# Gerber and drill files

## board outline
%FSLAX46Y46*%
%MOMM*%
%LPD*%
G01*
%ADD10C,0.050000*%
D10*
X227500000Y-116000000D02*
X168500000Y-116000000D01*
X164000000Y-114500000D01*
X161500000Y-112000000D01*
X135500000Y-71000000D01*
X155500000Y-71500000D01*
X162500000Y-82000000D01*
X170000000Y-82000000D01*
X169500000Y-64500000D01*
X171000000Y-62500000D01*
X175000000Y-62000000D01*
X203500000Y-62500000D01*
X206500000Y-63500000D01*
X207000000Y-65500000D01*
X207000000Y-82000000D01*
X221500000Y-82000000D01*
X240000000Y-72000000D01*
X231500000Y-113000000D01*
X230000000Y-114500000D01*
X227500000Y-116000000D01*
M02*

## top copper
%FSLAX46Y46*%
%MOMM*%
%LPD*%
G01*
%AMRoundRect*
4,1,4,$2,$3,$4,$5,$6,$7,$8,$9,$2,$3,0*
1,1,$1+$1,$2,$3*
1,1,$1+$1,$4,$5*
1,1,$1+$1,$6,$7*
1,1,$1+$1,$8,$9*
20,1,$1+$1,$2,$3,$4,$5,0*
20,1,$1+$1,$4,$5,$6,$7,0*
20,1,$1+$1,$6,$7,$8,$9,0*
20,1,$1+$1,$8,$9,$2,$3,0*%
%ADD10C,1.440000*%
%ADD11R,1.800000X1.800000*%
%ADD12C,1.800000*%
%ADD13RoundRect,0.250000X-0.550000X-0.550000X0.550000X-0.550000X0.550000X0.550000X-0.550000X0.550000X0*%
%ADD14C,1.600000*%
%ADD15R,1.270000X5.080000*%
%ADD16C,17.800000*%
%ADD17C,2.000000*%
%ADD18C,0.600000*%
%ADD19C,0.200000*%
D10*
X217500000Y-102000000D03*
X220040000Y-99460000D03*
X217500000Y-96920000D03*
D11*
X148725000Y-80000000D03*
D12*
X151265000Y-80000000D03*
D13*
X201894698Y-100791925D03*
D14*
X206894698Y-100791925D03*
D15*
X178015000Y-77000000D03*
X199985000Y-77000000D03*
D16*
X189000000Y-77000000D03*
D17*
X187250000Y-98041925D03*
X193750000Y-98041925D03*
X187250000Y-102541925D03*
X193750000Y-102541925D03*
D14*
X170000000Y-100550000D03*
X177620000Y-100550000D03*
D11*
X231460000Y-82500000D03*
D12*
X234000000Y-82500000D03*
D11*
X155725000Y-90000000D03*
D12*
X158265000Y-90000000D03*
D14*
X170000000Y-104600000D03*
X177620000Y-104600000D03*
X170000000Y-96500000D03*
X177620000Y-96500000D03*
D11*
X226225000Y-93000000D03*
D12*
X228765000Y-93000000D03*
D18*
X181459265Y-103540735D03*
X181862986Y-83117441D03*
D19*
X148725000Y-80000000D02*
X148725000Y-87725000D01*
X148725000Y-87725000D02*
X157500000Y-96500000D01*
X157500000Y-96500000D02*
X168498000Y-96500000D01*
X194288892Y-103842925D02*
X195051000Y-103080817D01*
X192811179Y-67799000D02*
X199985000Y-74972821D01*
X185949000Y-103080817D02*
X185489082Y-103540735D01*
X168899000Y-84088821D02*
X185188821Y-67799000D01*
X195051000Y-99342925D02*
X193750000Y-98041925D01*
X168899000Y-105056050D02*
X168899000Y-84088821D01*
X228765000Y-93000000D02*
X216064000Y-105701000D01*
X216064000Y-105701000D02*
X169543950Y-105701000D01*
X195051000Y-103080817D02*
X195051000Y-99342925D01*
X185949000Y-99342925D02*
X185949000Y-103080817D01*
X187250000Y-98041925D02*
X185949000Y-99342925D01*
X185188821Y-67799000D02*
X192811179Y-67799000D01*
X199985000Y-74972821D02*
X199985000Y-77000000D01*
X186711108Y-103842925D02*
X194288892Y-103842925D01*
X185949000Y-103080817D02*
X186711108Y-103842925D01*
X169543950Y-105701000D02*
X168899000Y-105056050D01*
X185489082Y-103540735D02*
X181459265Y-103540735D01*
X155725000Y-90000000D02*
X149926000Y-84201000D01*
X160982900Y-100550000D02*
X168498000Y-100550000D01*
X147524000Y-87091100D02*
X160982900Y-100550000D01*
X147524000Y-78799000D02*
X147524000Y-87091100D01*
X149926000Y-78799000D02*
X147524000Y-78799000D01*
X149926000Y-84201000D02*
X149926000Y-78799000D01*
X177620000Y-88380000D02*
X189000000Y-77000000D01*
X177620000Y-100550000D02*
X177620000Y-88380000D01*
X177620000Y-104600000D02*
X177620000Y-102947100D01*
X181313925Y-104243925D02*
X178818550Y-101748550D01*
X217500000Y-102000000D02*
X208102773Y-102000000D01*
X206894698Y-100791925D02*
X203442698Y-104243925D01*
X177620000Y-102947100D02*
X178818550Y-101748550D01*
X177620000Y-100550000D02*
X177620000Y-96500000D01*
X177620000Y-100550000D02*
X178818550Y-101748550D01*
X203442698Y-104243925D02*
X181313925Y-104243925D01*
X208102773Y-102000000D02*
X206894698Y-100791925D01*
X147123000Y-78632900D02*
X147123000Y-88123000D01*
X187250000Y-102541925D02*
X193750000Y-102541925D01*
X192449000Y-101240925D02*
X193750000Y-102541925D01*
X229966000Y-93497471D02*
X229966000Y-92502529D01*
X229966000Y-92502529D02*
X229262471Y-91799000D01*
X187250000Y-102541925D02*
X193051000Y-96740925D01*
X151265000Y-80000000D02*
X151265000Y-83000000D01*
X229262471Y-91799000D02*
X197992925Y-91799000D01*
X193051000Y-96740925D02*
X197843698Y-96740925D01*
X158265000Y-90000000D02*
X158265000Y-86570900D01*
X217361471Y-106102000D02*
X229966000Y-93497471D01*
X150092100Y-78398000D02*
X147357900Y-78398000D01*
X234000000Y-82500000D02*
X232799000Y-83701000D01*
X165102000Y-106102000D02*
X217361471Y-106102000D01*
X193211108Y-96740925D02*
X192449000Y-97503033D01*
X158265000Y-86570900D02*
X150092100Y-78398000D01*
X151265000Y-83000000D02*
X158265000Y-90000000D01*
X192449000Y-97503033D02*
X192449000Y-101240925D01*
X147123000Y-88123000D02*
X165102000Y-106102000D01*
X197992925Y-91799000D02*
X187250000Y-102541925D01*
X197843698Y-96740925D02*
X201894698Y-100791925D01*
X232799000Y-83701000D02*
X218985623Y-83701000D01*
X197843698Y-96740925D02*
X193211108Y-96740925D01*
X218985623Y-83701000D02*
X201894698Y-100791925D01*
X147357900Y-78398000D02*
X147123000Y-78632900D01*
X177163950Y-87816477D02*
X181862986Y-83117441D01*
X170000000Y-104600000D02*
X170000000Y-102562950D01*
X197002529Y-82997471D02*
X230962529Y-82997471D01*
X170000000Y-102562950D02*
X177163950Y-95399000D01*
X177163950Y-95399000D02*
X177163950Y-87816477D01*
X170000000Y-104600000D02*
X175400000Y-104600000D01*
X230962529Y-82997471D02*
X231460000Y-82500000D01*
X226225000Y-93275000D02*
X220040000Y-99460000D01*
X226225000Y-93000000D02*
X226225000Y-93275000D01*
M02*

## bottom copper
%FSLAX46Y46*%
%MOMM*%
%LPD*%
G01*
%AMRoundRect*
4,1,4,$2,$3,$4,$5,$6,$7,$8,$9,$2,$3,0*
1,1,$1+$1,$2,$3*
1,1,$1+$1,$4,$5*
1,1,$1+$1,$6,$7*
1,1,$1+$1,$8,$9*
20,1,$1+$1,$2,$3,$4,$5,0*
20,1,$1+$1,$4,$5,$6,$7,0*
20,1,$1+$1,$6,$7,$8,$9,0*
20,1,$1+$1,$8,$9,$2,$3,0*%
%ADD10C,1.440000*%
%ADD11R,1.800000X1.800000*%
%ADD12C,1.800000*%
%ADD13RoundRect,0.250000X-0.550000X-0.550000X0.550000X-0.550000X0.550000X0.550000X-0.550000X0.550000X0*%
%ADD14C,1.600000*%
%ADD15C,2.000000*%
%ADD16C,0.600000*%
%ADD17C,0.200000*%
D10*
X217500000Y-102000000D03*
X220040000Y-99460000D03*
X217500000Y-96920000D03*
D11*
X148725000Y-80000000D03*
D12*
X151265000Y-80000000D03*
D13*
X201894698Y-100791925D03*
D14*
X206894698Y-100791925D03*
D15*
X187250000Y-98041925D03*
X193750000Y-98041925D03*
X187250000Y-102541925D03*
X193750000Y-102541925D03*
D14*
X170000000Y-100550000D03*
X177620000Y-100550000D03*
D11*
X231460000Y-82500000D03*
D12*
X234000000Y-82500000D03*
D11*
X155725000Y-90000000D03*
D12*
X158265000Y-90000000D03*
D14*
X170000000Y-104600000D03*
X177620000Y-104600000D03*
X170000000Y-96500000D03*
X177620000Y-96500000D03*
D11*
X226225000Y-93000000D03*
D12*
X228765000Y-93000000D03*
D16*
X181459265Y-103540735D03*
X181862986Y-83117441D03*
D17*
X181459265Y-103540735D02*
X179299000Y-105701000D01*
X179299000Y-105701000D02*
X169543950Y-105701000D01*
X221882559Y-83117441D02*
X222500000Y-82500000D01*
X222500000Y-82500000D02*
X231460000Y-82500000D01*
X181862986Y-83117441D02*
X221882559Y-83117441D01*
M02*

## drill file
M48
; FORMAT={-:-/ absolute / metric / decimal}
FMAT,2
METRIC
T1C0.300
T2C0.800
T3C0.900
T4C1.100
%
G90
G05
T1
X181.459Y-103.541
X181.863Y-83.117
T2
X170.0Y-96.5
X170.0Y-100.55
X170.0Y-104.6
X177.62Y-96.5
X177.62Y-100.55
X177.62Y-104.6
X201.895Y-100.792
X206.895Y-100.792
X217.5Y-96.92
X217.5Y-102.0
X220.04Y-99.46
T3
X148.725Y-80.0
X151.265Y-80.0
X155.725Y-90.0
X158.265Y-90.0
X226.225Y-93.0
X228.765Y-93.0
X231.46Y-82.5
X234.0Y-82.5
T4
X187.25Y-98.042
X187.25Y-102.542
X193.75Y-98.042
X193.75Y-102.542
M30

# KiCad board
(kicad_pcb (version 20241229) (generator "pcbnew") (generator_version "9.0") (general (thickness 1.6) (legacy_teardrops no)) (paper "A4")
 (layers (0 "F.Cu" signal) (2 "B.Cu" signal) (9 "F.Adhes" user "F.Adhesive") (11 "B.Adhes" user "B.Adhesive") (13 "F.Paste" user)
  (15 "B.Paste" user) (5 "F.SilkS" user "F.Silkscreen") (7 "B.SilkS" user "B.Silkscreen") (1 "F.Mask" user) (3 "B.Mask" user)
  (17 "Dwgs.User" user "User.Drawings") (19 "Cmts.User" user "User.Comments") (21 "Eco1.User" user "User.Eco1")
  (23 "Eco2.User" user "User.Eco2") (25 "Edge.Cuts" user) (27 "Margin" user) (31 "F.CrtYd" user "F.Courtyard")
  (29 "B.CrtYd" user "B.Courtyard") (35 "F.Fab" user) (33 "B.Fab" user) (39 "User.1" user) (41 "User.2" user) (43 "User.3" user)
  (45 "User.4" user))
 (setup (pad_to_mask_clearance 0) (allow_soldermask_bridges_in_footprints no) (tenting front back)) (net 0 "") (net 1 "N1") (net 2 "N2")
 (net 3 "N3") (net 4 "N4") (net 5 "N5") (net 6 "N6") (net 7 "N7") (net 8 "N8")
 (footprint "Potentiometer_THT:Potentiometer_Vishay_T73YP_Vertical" (layer "F.Cu") (at 217.5 102)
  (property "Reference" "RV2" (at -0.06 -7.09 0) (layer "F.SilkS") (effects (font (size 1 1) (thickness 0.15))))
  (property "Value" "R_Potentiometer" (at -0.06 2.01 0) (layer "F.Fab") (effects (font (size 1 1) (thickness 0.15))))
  (pad "1" thru_hole circle (at 0 0) (size 1.44 1.44) (drill 0.8) (layers "*.Cu" "*.Mask") (remove_unused_layers no) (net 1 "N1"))
  (pad "2" thru_hole circle (at 2.54 -2.54) (size 1.44 1.44) (drill 0.8) (layers "*.Cu" "*.Mask") (remove_unused_layers no) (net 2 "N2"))
  (pad "3" thru_hole circle (at 0 -5.08) (size 1.44 1.44) (drill 0.8) (layers "*.Cu" "*.Mask") (remove_unused_layers no) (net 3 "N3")))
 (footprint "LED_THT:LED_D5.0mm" (layer "F.Cu") (at 148.725 80)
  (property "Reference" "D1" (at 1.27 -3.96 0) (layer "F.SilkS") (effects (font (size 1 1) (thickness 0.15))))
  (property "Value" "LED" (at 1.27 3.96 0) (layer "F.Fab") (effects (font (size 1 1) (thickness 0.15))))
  (pad "1" thru_hole rect (at 0 0) (size 1.8 1.8) (drill 0.9) (layers "*.Cu" "*.Mask") (remove_unused_layers no) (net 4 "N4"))
  (pad "2" thru_hole circle (at 2.54 0) (size 1.8 1.8) (drill 0.9) (layers "*.Cu" "*.Mask") (remove_unused_layers no) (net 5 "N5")))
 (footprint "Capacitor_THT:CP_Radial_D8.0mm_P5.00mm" (layer "F.Cu") (at 201.894698 100.791925)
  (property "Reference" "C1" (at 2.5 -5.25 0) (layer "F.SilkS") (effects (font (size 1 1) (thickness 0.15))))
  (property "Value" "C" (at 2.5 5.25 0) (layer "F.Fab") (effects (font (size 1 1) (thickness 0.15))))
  (pad "1" thru_hole roundrect (at 0 0) (size 1.6 1.6) (drill 0.8) (layers "*.Cu" "*.Mask") (remove_unused_layers no)
   (roundrect_rratio 0.15625) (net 5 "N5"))
  (pad "2" thru_hole circle (at 5 0) (size 1.6 1.6) (drill 0.8) (layers "*.Cu" "*.Mask") (remove_unused_layers no) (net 1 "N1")))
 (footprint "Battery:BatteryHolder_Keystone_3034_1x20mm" (layer "F.Cu") (at 189 77)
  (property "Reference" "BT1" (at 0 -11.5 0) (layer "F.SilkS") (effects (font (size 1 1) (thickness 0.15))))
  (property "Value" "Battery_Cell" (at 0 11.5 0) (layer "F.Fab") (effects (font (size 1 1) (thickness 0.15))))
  (pad "1" smd rect (at -10.985 0) (size 1.27 5.08) (layers "F.Cu" "F.Mask" "F.Paste") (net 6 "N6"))
  (pad "1" smd rect (at 10.985 0) (size 1.27 5.08) (layers "F.Cu" "F.Mask" "F.Paste") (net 6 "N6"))
  (pad "2" smd circle (at 0 0) (size 17.8 17.8) (layers "F.Cu" "F.Mask") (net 1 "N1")))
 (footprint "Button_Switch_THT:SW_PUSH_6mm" (layer "F.Cu") (at 187.25 98.041925)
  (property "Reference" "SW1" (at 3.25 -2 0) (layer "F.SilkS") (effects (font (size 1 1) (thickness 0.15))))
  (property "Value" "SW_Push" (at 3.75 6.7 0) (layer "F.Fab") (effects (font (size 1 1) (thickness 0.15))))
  (pad "1" thru_hole circle (at 0 0 90) (size 2 2) (drill 1.1) (layers "*.Cu" "*.Mask") (remove_unused_layers no) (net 6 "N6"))
  (pad "1" thru_hole circle (at 6.5 0 90) (size 2 2) (drill 1.1) (layers "*.Cu" "*.Mask") (remove_unused_layers no) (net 6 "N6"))
  (pad "2" thru_hole circle (at 0 4.5 90) (size 2 2) (drill 1.1) (layers "*.Cu" "*.Mask") (remove_unused_layers no) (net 5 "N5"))
  (pad "2" thru_hole circle (at 6.5 4.5 90) (size 2 2) (drill 1.1) (layers "*.Cu" "*.Mask") (remove_unused_layers no) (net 5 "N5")))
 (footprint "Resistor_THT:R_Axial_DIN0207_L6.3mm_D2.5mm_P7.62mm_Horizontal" (layer "F.Cu") (at 170 100.55)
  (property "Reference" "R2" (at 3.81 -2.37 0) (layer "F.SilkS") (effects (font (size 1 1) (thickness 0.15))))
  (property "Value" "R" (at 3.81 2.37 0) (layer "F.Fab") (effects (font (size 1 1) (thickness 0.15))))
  (pad "1" thru_hole circle (at 0 0) (size 1.6 1.6) (drill 0.8) (layers "*.Cu" "*.Mask") (remove_unused_layers no) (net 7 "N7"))
  (pad "2" thru_hole circle (at 7.62 0) (size 1.6 1.6) (drill 0.8) (layers "*.Cu" "*.Mask") (remove_unused_layers no) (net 1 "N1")))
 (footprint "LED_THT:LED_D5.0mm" (layer "F.Cu") (at 231.46 82.5)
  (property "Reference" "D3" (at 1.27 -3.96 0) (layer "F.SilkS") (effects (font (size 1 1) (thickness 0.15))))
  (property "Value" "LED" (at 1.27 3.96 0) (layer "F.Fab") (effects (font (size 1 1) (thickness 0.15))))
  (pad "1" thru_hole rect (at 0 0) (size 1.8 1.8) (drill 0.9) (layers "*.Cu" "*.Mask") (remove_unused_layers no) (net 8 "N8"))
  (pad "2" thru_hole circle (at 2.54 0) (size 1.8 1.8) (drill 0.9) (layers "*.Cu" "*.Mask") (remove_unused_layers no) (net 5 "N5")))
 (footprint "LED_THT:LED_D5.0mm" (layer "F.Cu") (at 155.725 90)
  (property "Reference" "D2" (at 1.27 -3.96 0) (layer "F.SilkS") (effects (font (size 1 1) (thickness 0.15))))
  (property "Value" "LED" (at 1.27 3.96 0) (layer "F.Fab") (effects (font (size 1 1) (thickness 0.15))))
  (pad "1" thru_hole rect (at 0 0) (size 1.8 1.8) (drill 0.9) (layers "*.Cu" "*.Mask") (remove_unused_layers no) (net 7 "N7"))
  (pad "2" thru_hole circle (at 2.54 0) (size 1.8 1.8) (drill 0.9) (layers "*.Cu" "*.Mask") (remove_unused_layers no) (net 5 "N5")))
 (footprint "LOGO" (layer "F.Cu") (at 175.5 67)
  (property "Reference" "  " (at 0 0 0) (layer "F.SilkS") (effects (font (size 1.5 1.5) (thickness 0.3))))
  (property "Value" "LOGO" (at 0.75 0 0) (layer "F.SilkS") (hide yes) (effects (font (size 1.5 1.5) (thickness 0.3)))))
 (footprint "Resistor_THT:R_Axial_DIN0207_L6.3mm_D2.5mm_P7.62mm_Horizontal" (layer "F.Cu") (at 170 104.6)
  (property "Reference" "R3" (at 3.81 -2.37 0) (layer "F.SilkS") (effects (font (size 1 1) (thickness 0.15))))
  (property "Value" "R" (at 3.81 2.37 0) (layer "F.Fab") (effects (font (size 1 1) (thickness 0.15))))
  (pad "1" thru_hole circle (at 0 0) (size 1.6 1.6) (drill 0.8) (layers "*.Cu" "*.Mask") (remove_unused_layers no) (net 8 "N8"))
  (pad "2" thru_hole circle (at 7.62 0) (size 1.6 1.6) (drill 0.8) (layers "*.Cu" "*.Mask") (remove_unused_layers no) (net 1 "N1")))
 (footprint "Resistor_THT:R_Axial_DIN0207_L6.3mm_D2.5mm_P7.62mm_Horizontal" (layer "F.Cu") (at 170 96.5)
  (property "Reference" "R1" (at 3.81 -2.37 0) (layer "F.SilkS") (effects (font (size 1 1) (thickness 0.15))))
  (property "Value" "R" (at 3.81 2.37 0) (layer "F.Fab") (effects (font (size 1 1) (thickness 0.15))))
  (pad "1" thru_hole circle (at 0 0) (size 1.6 1.6) (drill 0.8) (layers "*.Cu" "*.Mask") (remove_unused_layers no) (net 4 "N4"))
  (pad "2" thru_hole circle (at 7.62 0) (size 1.6 1.6) (drill 0.8) (layers "*.Cu" "*.Mask") (remove_unused_layers no) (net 1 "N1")))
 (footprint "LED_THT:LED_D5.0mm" (layer "F.Cu") (at 226.225 93)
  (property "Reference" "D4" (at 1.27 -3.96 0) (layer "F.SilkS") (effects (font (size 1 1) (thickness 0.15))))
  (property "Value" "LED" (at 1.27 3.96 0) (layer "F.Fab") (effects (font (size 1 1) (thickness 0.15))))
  (pad "1" thru_hole rect (at 0 0) (size 1.8 1.8) (drill 0.9) (layers "*.Cu" "*.Mask") (remove_unused_layers no) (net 2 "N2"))
  (pad "2" thru_hole circle (at 2.54 0) (size 1.8 1.8) (drill 0.9) (layers "*.Cu" "*.Mask") (remove_unused_layers no) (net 6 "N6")))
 (gr_poly
  (pts (xy 227.5 116) (xy 168.5 116) (xy 164 114.5) (xy 161.5 112) (xy 135.5 71) (xy 155.5 71.5) (xy 162.5 82) (xy 170 82) (xy 169.5 64.5)
   (xy 171 62.5) (xy 175 62) (xy 203.5 62.5) (xy 206.5 63.5) (xy 207 65.5) (xy 207 82) (xy 221.5 82) (xy 240 72) (xy 231.5 113)
   (xy 230 114.5))
  (stroke (width 0.05) (type solid)) (fill no) (layer "Edge.Cuts"))
 (segment (start 148.725 80) (end 148.725 87.725) (width 0.2) (layer "F.Cu") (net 4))
 (segment (start 148.725 87.725) (end 157.5 96.5) (width 0.2) (layer "F.Cu") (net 4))
 (segment (start 157.5 96.5) (end 168.498 96.5) (width 0.2) (layer "F.Cu") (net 4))
 (segment (start 194.288892 103.842925) (end 195.051 103.080817) (width 0.2) (layer "F.Cu") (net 6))
 (segment (start 192.811179 67.799) (end 199.985 74.972821) (width 0.2) (layer "F.Cu") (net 6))
 (segment (start 185.949 103.080817) (end 185.489082 103.540735) (width 0.2) (layer "F.Cu") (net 6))
 (segment (start 168.899 84.088821) (end 185.188821 67.799) (width 0.2) (layer "F.Cu") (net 6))
 (segment (start 195.051 99.342925) (end 193.75 98.041925) (width 0.2) (layer "F.Cu") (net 6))
 (segment (start 168.899 105.05605) (end 168.899 84.088821) (width 0.2) (layer "F.Cu") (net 6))
 (segment (start 228.765 93) (end 216.064 105.701) (width 0.2) (layer "F.Cu") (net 6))
 (segment (start 216.064 105.701) (end 169.54395 105.701) (width 0.2) (layer "F.Cu") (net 6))
 (segment (start 195.051 103.080817) (end 195.051 99.342925) (width 0.2) (layer "F.Cu") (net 6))
 (segment (start 185.949 99.342925) (end 185.949 103.080817) (width 0.2) (layer "F.Cu") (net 6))
 (segment (start 187.25 98.041925) (end 185.949 99.342925) (width 0.2) (layer "F.Cu") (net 6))
 (segment (start 185.188821 67.799) (end 192.811179 67.799) (width 0.2) (layer "F.Cu") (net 6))
 (segment (start 199.985 74.972821) (end 199.985 77) (width 0.2) (layer "F.Cu") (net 6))
 (segment (start 186.711108 103.842925) (end 194.288892 103.842925) (width 0.2) (layer "F.Cu") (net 6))
 (segment (start 185.949 103.080817) (end 186.711108 103.842925) (width 0.2) (layer "F.Cu") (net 6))
 (segment (start 169.54395 105.701) (end 168.899 105.05605) (width 0.2) (layer "F.Cu") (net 6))
 (segment (start 185.489082 103.540735) (end 181.459265 103.540735) (width 0.2) (layer "F.Cu") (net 6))
 (via (at 181.459265 103.540735) (size 0.6) (drill 0.3) (layers "F.Cu" "B.Cu") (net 6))
 (segment (start 181.459265 103.540735) (end 179.299 105.701) (width 0.2) (layer "B.Cu") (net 6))
 (segment (start 179.299 105.701) (end 169.54395 105.701) (width 0.2) (layer "B.Cu") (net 6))
 (segment (start 155.725 90) (end 149.926 84.201) (width 0.2) (layer "F.Cu") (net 7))
 (segment (start 160.9829 100.55) (end 168.498 100.55) (width 0.2) (layer "F.Cu") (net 7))
 (segment (start 147.524 87.0911) (end 160.9829 100.55) (width 0.2) (layer "F.Cu") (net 7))
 (segment (start 147.524 78.799) (end 147.524 87.0911) (width 0.2) (layer "F.Cu") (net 7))
 (segment (start 149.926 78.799) (end 147.524 78.799) (width 0.2) (layer "F.Cu") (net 7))
 (segment (start 149.926 84.201) (end 149.926 78.799) (width 0.2) (layer "F.Cu") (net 7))
 (segment (start 177.62 88.38) (end 189 77) (width 0.2) (layer "F.Cu") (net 1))
 (segment (start 177.62 100.55) (end 177.62 88.38) (width 0.2) (layer "F.Cu") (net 1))
 (segment (start 177.62 104.6) (end 177.62 102.9471) (width 0.2) (layer "F.Cu") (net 1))
 (segment (start 181.313925 104.243925) (end 178.81855 101.74855) (width 0.2) (layer "F.Cu") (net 1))
 (segment (start 217.5 102) (end 208.102773 102) (width 0.2) (layer "F.Cu") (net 1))
 (segment (start 206.894698 100.791925) (end 203.442698 104.243925) (width 0.2) (layer "F.Cu") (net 1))
 (segment (start 177.62 102.9471) (end 178.81855 101.74855) (width 0.2) (layer "F.Cu") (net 1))
 (segment (start 177.62 100.55) (end 177.62 96.5) (width 0.2) (layer "F.Cu") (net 1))
 (segment (start 177.62 100.55) (end 178.81855 101.74855) (width 0.2) (layer "F.Cu") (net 1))
 (segment (start 203.442698 104.243925) (end 181.313925 104.243925) (width 0.2) (layer "F.Cu") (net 1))
 (segment (start 208.102773 102) (end 206.894698 100.791925) (width 0.2) (layer "F.Cu") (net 1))
 (segment (start 147.123 78.6329) (end 147.123 88.123) (width 0.2) (layer "F.Cu") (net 5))
 (segment (start 187.25 102.541925) (end 193.75 102.541925) (width 0.2) (layer "F.Cu") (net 5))
 (segment (start 192.449 101.240925) (end 193.75 102.541925) (width 0.2) (layer "F.Cu") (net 5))
 (segment (start 229.966 93.497471) (end 229.966 92.502529) (width 0.2) (layer "F.Cu") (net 5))
 (segment (start 229.966 92.502529) (end 229.262471 91.799) (width 0.2) (layer "F.Cu") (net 5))
 (segment (start 187.25 102.541925) (end 193.051 96.740925) (width 0.2) (layer "F.Cu") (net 5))
 (segment (start 151.265 80) (end 151.265 83) (width 0.2) (layer "F.Cu") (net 5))
 (segment (start 229.262471 91.799) (end 197.992925 91.799) (width 0.2) (layer "F.Cu") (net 5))
 (segment (start 193.051 96.740925) (end 197.843698 96.740925) (width 0.2) (layer "F.Cu") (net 5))
 (segment (start 158.265 90) (end 158.265 86.5709) (width 0.2) (layer "F.Cu") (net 5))
 (segment (start 217.361471 106.102) (end 229.966 93.497471) (width 0.2) (layer "F.Cu") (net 5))
 (segment (start 150.0921 78.398) (end 147.3579 78.398) (width 0.2) (layer "F.Cu") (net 5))
 (segment (start 234 82.5) (end 232.799 83.701) (width 0.2) (layer "F.Cu") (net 5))
 (segment (start 165.102 106.102) (end 217.361471 106.102) (width 0.2) (layer "F.Cu") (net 5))
 (segment (start 193.211108 96.740925) (end 192.449 97.503033) (width 0.2) (layer "F.Cu") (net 5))
 (segment (start 158.265 86.5709) (end 150.0921 78.398) (width 0.2) (layer "F.Cu") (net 5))
 (segment (start 151.265 83) (end 158.265 90) (width 0.2) (layer "F.Cu") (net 5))
 (segment (start 192.449 97.503033) (end 192.449 101.240925) (width 0.2) (layer "F.Cu") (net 5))
 (segment (start 147.123 88.123) (end 165.102 106.102) (width 0.2) (layer "F.Cu") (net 5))
 (segment (start 197.992925 91.799) (end 187.25 102.541925) (width 0.2) (layer "F.Cu") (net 5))
 (segment (start 197.843698 96.740925) (end 201.894698 100.791925) (width 0.2) (layer "F.Cu") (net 5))
 (segment (start 232.799 83.701) (end 218.985623 83.701) (width 0.2) (layer "F.Cu") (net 5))
 (segment (start 197.843698 96.740925) (end 193.211108 96.740925) (width 0.2) (layer "F.Cu") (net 5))
 (segment (start 218.985623 83.701) (end 201.894698 100.791925) (width 0.2) (layer "F.Cu") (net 5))
 (segment (start 147.3579 78.398) (end 147.123 78.6329) (width 0.2) (layer "F.Cu") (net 5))
 (segment (start 177.16395 87.816477) (end 181.862986 83.117441) (width 0.2) (layer "F.Cu") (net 8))
 (segment (start 170 104.6) (end 170 102.56295) (width 0.2) (layer "F.Cu") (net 8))
 (segment (start 197.002529 82.997471) (end 230.962529 82.997471) (width 0.2) (layer "F.Cu") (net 8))
 (segment (start 170 102.56295) (end 177.16395 95.399) (width 0.2) (layer "F.Cu") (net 8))
 (segment (start 177.16395 95.399) (end 177.16395 87.816477) (width 0.2) (layer "F.Cu") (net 8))
 (segment (start 170 104.6) (end 175.4 104.6) (width 0.2) (layer "F.Cu") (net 8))
 (segment (start 230.962529 82.997471) (end 231.46 82.5) (width 0.2) (layer "F.Cu") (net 8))
 (via (at 181.862986 83.117441) (size 0.6) (drill 0.3) (layers "F.Cu" "B.Cu") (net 8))
 (segment (start 221.882559 83.117441) (end 222.5 82.5) (width 0.2) (layer "B.Cu") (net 8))
 (segment (start 222.5 82.5) (end 231.46 82.5) (width 0.2) (layer "B.Cu") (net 8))
 (segment (start 181.862986 83.117441) (end 221.882559 83.117441) (width 0.2) (layer "B.Cu") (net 8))
 (segment (start 226.225 93.275) (end 220.04 99.46) (width 0.2) (layer "F.Cu") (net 2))
 (segment (start 226.225 93) (end 226.225 93.275) (width 0.2) (layer "F.Cu") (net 2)))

